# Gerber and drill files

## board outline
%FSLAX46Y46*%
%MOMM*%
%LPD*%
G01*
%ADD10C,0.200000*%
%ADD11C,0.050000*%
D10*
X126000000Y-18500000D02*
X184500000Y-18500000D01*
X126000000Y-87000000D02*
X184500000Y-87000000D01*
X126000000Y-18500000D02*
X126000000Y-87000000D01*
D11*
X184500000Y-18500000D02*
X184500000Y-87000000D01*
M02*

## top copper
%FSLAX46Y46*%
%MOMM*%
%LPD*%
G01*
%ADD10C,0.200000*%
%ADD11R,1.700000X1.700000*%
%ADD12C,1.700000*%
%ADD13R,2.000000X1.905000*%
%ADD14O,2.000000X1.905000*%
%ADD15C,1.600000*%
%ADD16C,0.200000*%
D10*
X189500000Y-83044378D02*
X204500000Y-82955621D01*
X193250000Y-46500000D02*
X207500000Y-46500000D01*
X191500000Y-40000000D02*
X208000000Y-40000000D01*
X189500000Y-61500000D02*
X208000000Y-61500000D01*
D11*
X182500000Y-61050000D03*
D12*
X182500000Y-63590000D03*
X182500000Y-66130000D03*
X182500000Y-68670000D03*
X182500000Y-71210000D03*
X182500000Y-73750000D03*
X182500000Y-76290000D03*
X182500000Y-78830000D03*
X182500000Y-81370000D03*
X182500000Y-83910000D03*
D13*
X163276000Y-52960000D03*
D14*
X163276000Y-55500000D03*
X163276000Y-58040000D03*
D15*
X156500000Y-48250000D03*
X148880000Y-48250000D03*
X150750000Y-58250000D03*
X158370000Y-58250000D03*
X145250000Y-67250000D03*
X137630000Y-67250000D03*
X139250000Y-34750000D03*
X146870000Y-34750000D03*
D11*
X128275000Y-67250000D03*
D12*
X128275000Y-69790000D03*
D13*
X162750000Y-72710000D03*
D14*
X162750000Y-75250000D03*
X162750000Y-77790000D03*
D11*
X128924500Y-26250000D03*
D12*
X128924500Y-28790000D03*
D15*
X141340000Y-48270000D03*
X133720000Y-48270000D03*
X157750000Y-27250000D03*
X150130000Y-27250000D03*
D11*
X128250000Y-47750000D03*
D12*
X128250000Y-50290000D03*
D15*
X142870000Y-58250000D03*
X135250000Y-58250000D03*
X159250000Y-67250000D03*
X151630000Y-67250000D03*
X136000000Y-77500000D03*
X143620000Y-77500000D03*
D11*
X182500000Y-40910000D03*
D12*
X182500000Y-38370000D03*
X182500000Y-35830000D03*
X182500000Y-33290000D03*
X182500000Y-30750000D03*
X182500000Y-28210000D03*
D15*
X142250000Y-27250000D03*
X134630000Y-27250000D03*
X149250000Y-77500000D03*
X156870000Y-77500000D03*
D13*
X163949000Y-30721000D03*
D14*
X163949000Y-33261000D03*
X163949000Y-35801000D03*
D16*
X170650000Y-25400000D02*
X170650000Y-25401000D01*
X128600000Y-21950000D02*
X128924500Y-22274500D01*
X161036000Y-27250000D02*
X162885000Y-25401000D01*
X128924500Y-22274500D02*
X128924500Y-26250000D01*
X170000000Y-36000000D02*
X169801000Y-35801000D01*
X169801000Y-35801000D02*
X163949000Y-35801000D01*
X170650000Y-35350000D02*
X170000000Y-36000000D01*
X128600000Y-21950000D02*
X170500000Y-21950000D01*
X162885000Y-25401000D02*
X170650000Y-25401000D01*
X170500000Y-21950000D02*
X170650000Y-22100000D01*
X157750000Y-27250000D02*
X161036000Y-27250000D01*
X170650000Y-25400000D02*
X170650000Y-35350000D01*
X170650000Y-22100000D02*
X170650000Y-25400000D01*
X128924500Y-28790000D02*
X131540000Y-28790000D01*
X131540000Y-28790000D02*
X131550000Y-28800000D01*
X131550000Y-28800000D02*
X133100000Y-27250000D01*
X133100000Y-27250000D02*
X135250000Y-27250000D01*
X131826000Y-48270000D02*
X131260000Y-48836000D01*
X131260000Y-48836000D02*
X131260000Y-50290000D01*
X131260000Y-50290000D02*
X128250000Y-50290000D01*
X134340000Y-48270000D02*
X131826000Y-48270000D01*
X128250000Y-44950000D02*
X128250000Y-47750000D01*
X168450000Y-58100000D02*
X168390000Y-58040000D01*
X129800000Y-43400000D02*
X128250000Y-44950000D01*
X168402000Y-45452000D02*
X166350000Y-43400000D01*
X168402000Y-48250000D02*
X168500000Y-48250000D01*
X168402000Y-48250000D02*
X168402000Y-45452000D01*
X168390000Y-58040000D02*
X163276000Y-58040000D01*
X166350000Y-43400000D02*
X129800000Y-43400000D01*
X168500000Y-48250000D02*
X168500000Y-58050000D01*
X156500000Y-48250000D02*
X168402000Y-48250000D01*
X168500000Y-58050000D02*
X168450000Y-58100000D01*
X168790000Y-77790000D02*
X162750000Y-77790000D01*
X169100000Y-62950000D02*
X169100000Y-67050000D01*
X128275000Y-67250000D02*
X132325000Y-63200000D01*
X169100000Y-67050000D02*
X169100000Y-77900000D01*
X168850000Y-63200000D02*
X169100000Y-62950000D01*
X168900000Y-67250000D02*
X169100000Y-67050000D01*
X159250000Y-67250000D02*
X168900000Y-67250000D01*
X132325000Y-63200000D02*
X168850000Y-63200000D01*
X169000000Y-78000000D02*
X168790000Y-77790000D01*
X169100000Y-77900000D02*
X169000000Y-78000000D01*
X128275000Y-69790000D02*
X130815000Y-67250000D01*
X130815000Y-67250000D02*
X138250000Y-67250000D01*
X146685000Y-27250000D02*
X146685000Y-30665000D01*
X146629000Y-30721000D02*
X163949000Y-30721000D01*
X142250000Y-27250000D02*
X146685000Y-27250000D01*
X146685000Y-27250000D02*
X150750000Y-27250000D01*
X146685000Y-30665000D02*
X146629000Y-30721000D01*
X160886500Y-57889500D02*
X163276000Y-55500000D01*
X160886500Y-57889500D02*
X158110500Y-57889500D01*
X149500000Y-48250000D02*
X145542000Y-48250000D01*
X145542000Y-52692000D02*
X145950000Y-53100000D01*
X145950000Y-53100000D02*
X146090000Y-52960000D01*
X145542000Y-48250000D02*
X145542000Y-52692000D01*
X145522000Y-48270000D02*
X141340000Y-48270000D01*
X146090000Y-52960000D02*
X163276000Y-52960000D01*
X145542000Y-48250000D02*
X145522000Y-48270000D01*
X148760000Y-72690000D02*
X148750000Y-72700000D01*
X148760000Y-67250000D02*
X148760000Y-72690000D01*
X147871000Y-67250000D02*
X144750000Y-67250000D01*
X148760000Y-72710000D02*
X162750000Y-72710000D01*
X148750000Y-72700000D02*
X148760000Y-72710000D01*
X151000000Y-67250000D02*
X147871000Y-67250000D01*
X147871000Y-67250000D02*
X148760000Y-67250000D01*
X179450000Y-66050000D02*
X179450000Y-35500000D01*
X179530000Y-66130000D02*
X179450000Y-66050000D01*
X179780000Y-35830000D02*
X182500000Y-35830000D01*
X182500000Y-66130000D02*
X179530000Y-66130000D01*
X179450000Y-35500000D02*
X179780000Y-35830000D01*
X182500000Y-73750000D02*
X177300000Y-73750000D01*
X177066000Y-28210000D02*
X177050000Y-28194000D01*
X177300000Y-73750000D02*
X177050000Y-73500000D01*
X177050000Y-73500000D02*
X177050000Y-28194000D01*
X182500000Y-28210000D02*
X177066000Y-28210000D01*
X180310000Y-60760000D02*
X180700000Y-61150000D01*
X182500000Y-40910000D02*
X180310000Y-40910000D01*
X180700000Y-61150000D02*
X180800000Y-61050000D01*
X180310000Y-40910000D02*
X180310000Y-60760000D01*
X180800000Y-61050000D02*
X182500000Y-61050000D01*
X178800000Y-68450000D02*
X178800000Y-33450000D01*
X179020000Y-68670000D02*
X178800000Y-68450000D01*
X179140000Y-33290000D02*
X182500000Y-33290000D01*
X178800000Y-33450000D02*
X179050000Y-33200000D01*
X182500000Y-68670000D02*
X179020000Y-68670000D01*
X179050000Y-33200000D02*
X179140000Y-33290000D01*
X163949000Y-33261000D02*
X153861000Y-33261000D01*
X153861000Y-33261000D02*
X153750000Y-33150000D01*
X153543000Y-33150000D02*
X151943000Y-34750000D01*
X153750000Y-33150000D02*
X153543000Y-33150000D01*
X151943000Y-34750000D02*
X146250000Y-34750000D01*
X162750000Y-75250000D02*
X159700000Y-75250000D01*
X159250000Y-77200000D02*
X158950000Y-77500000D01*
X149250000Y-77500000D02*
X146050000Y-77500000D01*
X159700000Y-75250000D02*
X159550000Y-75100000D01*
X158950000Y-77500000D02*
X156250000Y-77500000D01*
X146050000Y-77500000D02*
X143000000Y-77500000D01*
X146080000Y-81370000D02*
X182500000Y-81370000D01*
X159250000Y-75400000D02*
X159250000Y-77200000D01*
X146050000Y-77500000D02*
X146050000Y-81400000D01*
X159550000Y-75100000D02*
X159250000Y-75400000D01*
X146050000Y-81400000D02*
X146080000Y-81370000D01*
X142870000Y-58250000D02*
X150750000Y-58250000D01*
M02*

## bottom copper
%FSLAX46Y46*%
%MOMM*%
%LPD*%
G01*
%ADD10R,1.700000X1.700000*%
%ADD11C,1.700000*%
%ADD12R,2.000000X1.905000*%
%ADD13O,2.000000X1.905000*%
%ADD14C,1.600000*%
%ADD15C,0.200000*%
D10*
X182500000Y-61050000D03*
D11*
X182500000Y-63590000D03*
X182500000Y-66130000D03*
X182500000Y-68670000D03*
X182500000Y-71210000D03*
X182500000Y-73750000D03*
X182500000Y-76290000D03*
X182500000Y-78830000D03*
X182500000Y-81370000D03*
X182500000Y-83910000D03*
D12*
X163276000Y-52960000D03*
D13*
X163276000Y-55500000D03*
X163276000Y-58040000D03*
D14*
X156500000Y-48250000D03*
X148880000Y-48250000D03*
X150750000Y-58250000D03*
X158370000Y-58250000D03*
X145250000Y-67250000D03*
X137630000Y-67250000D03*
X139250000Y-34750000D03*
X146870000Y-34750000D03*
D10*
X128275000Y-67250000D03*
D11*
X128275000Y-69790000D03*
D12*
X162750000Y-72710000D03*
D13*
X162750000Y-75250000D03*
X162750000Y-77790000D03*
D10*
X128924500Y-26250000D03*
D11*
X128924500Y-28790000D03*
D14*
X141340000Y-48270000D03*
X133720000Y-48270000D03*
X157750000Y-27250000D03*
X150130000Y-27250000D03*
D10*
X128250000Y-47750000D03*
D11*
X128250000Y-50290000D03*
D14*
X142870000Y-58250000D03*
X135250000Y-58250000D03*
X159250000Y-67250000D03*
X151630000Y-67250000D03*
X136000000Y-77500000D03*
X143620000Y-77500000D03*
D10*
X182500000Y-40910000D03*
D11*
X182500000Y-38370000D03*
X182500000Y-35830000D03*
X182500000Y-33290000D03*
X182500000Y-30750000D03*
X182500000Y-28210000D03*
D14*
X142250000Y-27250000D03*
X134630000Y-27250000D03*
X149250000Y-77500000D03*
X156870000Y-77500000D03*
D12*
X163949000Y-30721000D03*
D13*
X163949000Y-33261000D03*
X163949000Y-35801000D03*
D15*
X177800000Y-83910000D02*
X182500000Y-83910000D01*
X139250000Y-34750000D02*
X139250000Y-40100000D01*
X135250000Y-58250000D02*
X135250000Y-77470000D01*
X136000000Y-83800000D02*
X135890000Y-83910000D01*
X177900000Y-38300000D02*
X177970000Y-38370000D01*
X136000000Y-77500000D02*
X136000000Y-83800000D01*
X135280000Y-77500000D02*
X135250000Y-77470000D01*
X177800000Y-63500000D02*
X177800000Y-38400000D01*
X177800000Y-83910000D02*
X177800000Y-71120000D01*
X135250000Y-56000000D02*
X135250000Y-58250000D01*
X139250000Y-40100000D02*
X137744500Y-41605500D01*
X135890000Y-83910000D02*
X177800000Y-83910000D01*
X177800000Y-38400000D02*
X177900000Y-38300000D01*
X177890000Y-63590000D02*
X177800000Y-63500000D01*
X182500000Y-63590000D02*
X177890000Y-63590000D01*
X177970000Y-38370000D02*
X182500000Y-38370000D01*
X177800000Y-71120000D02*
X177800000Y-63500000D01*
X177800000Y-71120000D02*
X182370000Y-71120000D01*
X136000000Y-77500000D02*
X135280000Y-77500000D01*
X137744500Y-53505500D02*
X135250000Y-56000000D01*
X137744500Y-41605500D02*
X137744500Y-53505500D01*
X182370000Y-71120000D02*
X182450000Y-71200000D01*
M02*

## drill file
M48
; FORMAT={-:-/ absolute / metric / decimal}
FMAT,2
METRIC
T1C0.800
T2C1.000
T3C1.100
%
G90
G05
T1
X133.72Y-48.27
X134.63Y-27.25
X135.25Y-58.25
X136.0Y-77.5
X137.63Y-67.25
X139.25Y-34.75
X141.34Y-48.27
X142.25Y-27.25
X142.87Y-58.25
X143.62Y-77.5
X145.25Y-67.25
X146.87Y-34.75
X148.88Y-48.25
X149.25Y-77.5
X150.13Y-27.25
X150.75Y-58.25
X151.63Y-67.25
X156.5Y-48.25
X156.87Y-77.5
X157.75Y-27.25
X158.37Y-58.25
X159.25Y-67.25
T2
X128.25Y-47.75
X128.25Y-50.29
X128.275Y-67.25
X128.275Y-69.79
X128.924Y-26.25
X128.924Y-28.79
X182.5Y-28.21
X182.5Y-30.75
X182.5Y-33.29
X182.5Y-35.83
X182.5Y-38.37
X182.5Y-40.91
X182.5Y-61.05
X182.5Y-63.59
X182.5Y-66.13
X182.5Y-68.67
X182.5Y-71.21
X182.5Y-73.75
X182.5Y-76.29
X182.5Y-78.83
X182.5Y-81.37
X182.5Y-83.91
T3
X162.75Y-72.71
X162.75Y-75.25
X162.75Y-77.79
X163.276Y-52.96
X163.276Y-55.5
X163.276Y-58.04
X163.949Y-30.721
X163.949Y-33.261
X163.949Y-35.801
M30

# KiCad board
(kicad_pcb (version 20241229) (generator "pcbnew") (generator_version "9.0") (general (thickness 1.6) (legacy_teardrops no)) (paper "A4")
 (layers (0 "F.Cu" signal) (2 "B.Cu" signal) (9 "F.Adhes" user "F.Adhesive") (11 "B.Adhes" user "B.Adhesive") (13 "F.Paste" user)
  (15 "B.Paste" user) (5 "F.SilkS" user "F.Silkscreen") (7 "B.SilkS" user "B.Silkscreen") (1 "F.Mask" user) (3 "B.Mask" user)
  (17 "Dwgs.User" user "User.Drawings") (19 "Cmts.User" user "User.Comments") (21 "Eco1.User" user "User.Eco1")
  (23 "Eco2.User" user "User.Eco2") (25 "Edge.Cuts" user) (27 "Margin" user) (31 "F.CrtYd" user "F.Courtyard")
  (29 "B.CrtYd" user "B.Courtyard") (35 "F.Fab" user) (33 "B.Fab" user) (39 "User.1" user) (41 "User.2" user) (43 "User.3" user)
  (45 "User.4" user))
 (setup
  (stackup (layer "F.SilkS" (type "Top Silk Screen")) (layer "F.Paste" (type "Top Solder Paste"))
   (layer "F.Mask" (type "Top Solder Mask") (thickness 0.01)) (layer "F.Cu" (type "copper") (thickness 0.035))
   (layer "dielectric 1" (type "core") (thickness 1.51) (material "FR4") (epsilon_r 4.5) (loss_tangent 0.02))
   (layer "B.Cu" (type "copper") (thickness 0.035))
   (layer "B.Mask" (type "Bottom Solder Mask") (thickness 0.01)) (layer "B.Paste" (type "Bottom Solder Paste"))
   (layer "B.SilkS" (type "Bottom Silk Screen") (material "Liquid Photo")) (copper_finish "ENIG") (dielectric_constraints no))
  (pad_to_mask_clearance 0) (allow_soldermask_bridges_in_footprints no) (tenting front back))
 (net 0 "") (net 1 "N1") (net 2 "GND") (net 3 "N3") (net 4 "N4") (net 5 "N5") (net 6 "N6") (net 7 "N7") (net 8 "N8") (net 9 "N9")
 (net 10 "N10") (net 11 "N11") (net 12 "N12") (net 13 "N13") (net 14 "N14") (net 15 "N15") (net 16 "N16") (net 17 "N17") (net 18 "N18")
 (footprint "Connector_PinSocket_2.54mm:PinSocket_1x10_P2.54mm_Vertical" (layer "F.Cu") (at 182.5 61.05)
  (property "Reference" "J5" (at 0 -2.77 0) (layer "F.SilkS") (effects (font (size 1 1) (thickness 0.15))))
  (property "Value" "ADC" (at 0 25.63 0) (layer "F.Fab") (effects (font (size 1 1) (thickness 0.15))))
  (pad "1" thru_hole rect (at 0 0) (size 1.7 1.7) (drill 1) (layers "*.Cu" "*.Mask") (remove_unused_layers yes) (keep_end_layers yes)
   (zone_layer_connections) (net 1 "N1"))
  (pad "2" thru_hole circle (at 0 2.54) (size 1.7 1.7) (drill 1) (layers "*.Cu" "*.Mask") (remove_unused_layers yes) (keep_end_layers yes)
   (zone_layer_connections) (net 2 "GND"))
  (pad "3" thru_hole circle (at 0 5.08) (size 1.7 1.7) (drill 1) (layers "*.Cu" "*.Mask") (remove_unused_layers yes) (keep_end_layers yes)
   (zone_layer_connections) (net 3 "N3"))
  (pad "4" thru_hole circle (at 0 7.62) (size 1.7 1.7) (drill 1) (layers "*.Cu" "*.Mask") (remove_unused_layers yes) (keep_end_layers yes)
   (zone_layer_connections) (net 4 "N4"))
  (pad "5" thru_hole circle (at 0 10.16) (size 1.7 1.7) (drill 1) (layers "*.Cu" "*.Mask") (remove_unused_layers yes) (keep_end_layers yes)
   (zone_layer_connections) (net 2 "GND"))
  (pad "6" thru_hole circle (at 0 12.7) (size 1.7 1.7) (drill 1) (layers "*.Cu" "*.Mask") (remove_unused_layers yes) (keep_end_layers yes)
   (zone_layer_connections) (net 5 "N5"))
  (pad "7" thru_hole circle (at 0 15.24) (size 1.7 1.7) (drill 1) (layers "*.Cu" "*.Mask") (remove_unused_layers yes) (keep_end_layers yes)
   (zone_layer_connections) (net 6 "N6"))
  (pad "8" thru_hole circle (at 0 17.78) (size 1.7 1.7) (drill 1) (layers "*.Cu" "*.Mask") (remove_unused_layers yes) (keep_end_layers yes)
   (zone_layer_connections) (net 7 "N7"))
  (pad "9" thru_hole circle (at 0 20.32) (size 1.7 1.7) (drill 1) (layers "*.Cu" "*.Mask") (remove_unused_layers yes) (keep_end_layers yes)
   (zone_layer_connections) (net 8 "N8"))
  (pad "10" thru_hole circle (at 0 22.86) (size 1.7 1.7) (drill 1) (layers "*.Cu" "*.Mask") (remove_unused_layers yes) (keep_end_layers yes)
   (zone_layer_connections) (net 2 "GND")))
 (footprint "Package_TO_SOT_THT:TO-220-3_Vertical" (layer "F.Cu") (at 163.276 52.96 -90)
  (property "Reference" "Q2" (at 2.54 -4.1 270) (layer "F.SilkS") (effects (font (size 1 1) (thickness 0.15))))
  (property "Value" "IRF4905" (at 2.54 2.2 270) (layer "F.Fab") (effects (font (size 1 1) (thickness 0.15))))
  (pad "1" thru_hole rect (at 0 0 270) (size 1.905 2) (drill 1.1) (layers "*.Cu" "*.Mask") (remove_unused_layers yes) (keep_end_layers yes)
   (zone_layer_connections) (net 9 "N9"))
  (pad "2" thru_hole oval (at 2.54 0 270) (size 1.905 2) (drill 1.1) (layers "*.Cu" "*.Mask") (remove_unused_layers yes)
   (keep_end_layers yes) (zone_layer_connections) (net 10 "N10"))
  (pad "3" thru_hole oval (at 5.08 0 270) (size 1.905 2) (drill 1.1) (layers "*.Cu" "*.Mask") (remove_unused_layers yes)
   (keep_end_layers yes) (zone_layer_connections) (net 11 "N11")))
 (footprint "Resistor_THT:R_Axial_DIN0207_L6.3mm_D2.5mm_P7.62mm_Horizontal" (layer "F.Cu") (at 156.5 48.25 180)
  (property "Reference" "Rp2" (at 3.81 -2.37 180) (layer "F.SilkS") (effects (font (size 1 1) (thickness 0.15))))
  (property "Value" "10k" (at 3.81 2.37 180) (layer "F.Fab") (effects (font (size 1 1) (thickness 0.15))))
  (pad "1" thru_hole circle (at 0 0 180) (size 1.6 1.6) (drill 0.8) (layers "*.Cu" "*.Mask") (remove_unused_layers no) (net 11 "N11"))
  (pad "2" thru_hole circle (at 7.62 0 180) (size 1.6 1.6) (drill 0.8) (layers "*.Cu" "*.Mask") (remove_unused_layers no) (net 9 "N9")))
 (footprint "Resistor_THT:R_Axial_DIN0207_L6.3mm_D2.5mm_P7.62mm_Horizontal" (layer "F.Cu") (at 150.75 58.25)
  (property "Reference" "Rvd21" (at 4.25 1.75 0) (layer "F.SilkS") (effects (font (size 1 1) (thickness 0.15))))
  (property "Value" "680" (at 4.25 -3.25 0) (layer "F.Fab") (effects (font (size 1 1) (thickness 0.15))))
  (pad "1" thru_hole circle (at 0 0) (size 1.6 1.6) (drill 0.8) (layers "*.Cu" "*.Mask") (remove_unused_layers no) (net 7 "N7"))
  (pad "2" thru_hole circle (at 7.62 0) (size 1.6 1.6) (drill 0.8) (layers "*.Cu" "*.Mask") (remove_unused_layers no) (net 10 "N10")))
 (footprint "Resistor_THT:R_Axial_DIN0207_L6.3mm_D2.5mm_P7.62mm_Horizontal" (layer "F.Cu") (at 145.25 67.25 180)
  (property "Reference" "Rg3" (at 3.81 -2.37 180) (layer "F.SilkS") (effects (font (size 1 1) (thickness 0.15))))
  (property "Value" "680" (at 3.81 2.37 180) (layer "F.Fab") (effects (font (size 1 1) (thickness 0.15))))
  (pad "1" thru_hole circle (at 0 0 180) (size 1.6 1.6) (drill 0.8) (layers "*.Cu" "*.Mask") (remove_unused_layers no) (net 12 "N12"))
  (pad "2" thru_hole circle (at 7.62 0 180) (size 1.6 1.6) (drill 0.8) (layers "*.Cu" "*.Mask") (remove_unused_layers no) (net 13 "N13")))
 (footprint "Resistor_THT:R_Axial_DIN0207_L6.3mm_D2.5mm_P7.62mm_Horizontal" (layer "F.Cu") (at 139.25 34.75)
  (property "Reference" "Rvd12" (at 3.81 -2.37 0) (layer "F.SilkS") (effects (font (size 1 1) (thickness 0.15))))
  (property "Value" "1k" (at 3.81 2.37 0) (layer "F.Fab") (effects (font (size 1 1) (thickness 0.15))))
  (pad "1" thru_hole circle (at 0 0) (size 1.6 1.6) (drill 0.8) (layers "*.Cu" "*.Mask") (remove_unused_layers no) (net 2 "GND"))
  (pad "2" thru_hole circle (at 7.62 0) (size 1.6 1.6) (drill 0.8) (layers "*.Cu" "*.Mask") (remove_unused_layers no) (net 6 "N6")))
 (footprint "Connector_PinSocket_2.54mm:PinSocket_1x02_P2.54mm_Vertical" (layer "F.Cu") (at 128.275 67.25)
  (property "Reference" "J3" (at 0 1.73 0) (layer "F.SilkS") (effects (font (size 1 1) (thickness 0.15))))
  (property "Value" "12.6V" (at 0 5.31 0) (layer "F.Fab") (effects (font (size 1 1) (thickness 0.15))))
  (pad "1" thru_hole rect (at 0 0) (size 1.7 1.7) (drill 1) (layers "*.Cu" "*.Mask") (remove_unused_layers yes) (keep_end_layers yes)
   (zone_layer_connections) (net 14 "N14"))
  (pad "2" thru_hole circle (at 0 2.54) (size 1.7 1.7) (drill 1) (layers "*.Cu" "*.Mask") (remove_unused_layers yes) (keep_end_layers yes)
   (zone_layer_connections) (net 13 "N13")))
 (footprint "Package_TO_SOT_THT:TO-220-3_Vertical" (layer "F.Cu") (at 162.75 72.71 -90)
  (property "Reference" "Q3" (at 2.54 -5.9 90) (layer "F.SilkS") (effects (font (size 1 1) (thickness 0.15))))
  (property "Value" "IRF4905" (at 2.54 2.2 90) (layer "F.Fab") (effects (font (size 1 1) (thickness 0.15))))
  (pad "1" thru_hole rect (at 0 0 270) (size 1.905 2) (drill 1.1) (layers "*.Cu" "*.Mask") (remove_unused_layers yes) (keep_end_layers yes)
   (zone_layer_connections) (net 12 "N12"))
  (pad "2" thru_hole oval (at 2.54 0 270) (size 1.905 2) (drill 1.1) (layers "*.Cu" "*.Mask") (remove_unused_layers yes)
   (keep_end_layers yes) (zone_layer_connections) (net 8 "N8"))
  (pad "3" thru_hole oval (at 5.08 0 270) (size 1.905 2) (drill 1.1) (layers "*.Cu" "*.Mask") (remove_unused_layers yes)
   (keep_end_layers yes) (zone_layer_connections) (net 14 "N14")))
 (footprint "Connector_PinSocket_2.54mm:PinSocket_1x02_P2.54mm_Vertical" (layer "F.Cu") (at 128.9245 26.25)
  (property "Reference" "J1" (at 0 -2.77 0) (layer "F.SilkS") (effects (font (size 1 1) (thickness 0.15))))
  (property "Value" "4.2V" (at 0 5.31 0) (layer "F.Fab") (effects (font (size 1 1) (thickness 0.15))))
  (pad "1" thru_hole rect (at 0 0) (size 1.7 1.7) (drill 1) (layers "*.Cu" "*.Mask") (remove_unused_layers yes) (keep_end_layers yes)
   (zone_layer_connections) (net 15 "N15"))
  (pad "2" thru_hole circle (at 0 2.54) (size 1.7 1.7) (drill 1) (layers "*.Cu" "*.Mask") (remove_unused_layers yes) (keep_end_layers yes)
   (zone_layer_connections) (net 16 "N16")))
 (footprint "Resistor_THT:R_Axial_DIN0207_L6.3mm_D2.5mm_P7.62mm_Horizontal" (layer "F.Cu") (at 141.34 48.27 180)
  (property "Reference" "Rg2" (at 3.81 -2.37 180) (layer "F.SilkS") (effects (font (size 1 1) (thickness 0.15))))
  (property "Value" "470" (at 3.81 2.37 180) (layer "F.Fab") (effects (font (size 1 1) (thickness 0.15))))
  (pad "1" thru_hole circle (at 0 0 180) (size 1.6 1.6) (drill 0.8) (layers "*.Cu" "*.Mask") (remove_unused_layers no) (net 9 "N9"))
  (pad "2" thru_hole circle (at 7.62 0 180) (size 1.6 1.6) (drill 0.8) (layers "*.Cu" "*.Mask") (remove_unused_layers no) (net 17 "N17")))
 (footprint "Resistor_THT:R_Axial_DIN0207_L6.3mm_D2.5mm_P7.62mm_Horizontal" (layer "F.Cu") (at 157.75 27.25 180)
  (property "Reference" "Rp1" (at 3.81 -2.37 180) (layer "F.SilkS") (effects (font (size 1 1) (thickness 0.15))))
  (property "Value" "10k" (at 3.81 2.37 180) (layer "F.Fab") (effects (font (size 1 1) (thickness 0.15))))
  (pad "1" thru_hole circle (at 0 0 180) (size 1.6 1.6) (drill 0.8) (layers "*.Cu" "*.Mask") (remove_unused_layers no) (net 15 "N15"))
  (pad "2" thru_hole circle (at 7.62 0 180) (size 1.6 1.6) (drill 0.8) (layers "*.Cu" "*.Mask") (remove_unused_layers no) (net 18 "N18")))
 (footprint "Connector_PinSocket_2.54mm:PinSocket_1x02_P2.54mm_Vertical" (layer "F.Cu") (at 128.25 47.75)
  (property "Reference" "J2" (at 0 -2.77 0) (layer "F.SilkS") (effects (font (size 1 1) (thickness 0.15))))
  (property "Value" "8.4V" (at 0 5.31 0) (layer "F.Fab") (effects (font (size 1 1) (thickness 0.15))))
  (pad "1" thru_hole rect (at 0 0) (size 1.7 1.7) (drill 1) (layers "*.Cu" "*.Mask") (remove_unused_layers yes) (keep_end_layers yes)
   (zone_layer_connections) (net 11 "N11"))
  (pad "2" thru_hole circle (at 0 2.54) (size 1.7 1.7) (drill 1) (layers "*.Cu" "*.Mask") (remove_unused_layers yes) (keep_end_layers yes)
   (zone_layer_connections) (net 17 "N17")))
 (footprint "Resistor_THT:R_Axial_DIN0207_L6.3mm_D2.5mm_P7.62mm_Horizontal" (layer "F.Cu") (at 142.87 58.25 180)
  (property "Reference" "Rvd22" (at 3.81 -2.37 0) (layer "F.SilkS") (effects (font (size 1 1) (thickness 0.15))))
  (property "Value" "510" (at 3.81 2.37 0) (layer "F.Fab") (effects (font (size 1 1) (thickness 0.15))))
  (pad "1" thru_hole circle (at 0 0 180) (size 1.6 1.6) (drill 0.8) (layers "*.Cu" "*.Mask") (remove_unused_layers no) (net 7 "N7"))
  (pad "2" thru_hole circle (at 7.62 0 180) (size 1.6 1.6) (drill 0.8) (layers "*.Cu" "*.Mask") (remove_unused_layers no) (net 2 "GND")))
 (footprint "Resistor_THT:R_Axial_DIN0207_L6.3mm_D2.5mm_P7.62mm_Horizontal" (layer "F.Cu") (at 159.25 67.25 180)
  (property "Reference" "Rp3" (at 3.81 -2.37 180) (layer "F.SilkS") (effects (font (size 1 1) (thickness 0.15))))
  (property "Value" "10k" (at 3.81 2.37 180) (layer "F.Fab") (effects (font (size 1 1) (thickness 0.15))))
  (pad "1" thru_hole circle (at 0 0 180) (size 1.6 1.6) (drill 0.8) (layers "*.Cu" "*.Mask") (remove_unused_layers no) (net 14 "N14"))
  (pad "2" thru_hole circle (at 7.62 0 180) (size 1.6 1.6) (drill 0.8) (layers "*.Cu" "*.Mask") (remove_unused_layers no) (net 12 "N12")))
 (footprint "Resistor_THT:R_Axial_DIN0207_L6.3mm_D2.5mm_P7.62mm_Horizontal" (layer "F.Cu") (at 136 77.5)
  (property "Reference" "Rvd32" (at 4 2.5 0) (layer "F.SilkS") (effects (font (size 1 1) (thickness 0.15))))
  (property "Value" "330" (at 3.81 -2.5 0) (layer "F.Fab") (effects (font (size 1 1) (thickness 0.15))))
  (pad "1" thru_hole circle (at 0 0) (size 1.6 1.6) (drill 0.8) (layers "*.Cu" "*.Mask") (remove_unused_layers no) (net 2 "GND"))
  (pad "2" thru_hole circle (at 7.62 0) (size 1.6 1.6) (drill 0.8) (layers "*.Cu" "*.Mask") (remove_unused_layers no) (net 8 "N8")))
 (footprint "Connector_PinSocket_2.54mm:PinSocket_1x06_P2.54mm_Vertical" (layer "F.Cu") (at 182.5 40.91 180)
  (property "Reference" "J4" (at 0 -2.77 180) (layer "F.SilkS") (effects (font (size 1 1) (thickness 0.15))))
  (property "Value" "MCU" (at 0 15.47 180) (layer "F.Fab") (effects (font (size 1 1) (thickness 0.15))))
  (pad "1" thru_hole rect (at 0 0 180) (size 1.7 1.7) (drill 1) (layers "*.Cu" "*.Mask") (remove_unused_layers yes) (keep_end_layers yes)
   (zone_layer_connections) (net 1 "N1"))
  (pad "2" thru_hole circle (at 0 2.54 180) (size 1.7 1.7) (drill 1) (layers "*.Cu" "*.Mask") (remove_unused_layers yes)
   (keep_end_layers yes) (zone_layer_connections) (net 2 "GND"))
  (pad "3" thru_hole circle (at 0 5.08 180) (size 1.7 1.7) (drill 1) (layers "*.Cu" "*.Mask") (remove_unused_layers yes)
   (keep_end_layers yes) (zone_layer_connections) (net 3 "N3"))
  (pad "4" thru_hole circle (at 0 7.62 180) (size 1.7 1.7) (drill 1) (layers "*.Cu" "*.Mask") (remove_unused_layers yes)
   (keep_end_layers yes) (zone_layer_connections) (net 4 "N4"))
  (pad "5" thru_hole circle (at 0 10.16 180) (size 1.7 1.7) (drill 1) (layers "*.Cu" "*.Mask") (remove_unused_layers yes)
   (keep_end_layers yes) (zone_layer_connections) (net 2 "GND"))
  (pad "6" thru_hole circle (at 0 12.7 180) (size 1.7 1.7) (drill 1) (layers "*.Cu" "*.Mask") (remove_unused_layers yes)
   (keep_end_layers yes) (zone_layer_connections) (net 5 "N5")))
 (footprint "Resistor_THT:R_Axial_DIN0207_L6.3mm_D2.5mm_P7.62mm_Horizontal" (layer "F.Cu") (at 142.25 27.25 180)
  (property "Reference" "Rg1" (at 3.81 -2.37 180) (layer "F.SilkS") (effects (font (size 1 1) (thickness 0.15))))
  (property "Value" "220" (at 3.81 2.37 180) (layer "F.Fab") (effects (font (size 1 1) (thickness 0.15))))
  (pad "1" thru_hole circle (at 0 0 180) (size 1.6 1.6) (drill 0.8) (layers "*.Cu" "*.Mask") (remove_unused_layers no) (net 18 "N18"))
  (pad "2" thru_hole circle (at 7.62 0 180) (size 1.6 1.6) (drill 0.8) (layers "*.Cu" "*.Mask") (remove_unused_layers no) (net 16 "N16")))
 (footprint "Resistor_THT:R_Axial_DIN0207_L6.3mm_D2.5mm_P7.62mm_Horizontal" (layer "F.Cu") (at 149.25 77.5)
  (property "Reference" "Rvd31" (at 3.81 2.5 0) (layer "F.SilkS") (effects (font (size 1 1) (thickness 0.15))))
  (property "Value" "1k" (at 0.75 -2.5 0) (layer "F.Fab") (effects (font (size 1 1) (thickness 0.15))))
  (pad "1" thru_hole circle (at 0 0) (size 1.6 1.6) (drill 0.8) (layers "*.Cu" "*.Mask") (remove_unused_layers no) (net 8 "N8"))
  (pad "2" thru_hole circle (at 7.62 0) (size 1.6 1.6) (drill 0.8) (layers "*.Cu" "*.Mask") (remove_unused_layers no) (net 8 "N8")))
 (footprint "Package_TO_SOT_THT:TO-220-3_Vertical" (layer "F.Cu") (at 163.949 30.721 -90)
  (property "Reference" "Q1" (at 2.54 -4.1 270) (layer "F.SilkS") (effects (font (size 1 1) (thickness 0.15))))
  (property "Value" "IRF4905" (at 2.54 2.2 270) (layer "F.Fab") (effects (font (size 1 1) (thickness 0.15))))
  (pad "1" thru_hole rect (at 0 0 270) (size 1.905 2) (drill 1.1) (layers "*.Cu" "*.Mask") (remove_unused_layers yes) (keep_end_layers yes)
   (zone_layer_connections) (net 18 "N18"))
  (pad "2" thru_hole oval (at 2.54 0 270) (size 1.905 2) (drill 1.1) (layers "*.Cu" "*.Mask") (remove_unused_layers yes)
   (keep_end_layers yes) (zone_layer_connections) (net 6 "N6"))
  (pad "3" thru_hole oval (at 5.08 0 270) (size 1.905 2) (drill 1.1) (layers "*.Cu" "*.Mask") (remove_unused_layers yes)
   (keep_end_layers yes) (zone_layer_connections) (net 15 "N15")))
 (gr_line (start 189.5 83.044378) (end 204.5 82.955621) (stroke (width 0.2) (type default)) (layer "F.Cu"))
 (gr_line (start 193.25 46.5) (end 207.5 46.5) (stroke (width 0.2) (type default)) (layer "F.Cu"))
 (gr_line (start 191.5 40) (end 208 40) (stroke (width 0.2) (type default)) (layer "F.Cu"))
 (gr_line (start 189.5 61.5) (end 208 61.5) (stroke (width 0.2) (type default)) (layer "F.Cu"))
 (gr_line (start 126 18.5) (end 184.5 18.5) (stroke (width 0.2) (type solid)) (layer "Edge.Cuts"))
 (gr_line (start 126 87) (end 184.5 87) (stroke (width 0.2) (type solid)) (layer "Edge.Cuts"))
 (gr_line (start 126 18.5) (end 126 87) (stroke (width 0.2) (type solid)) (layer "Edge.Cuts"))
 (gr_line (start 184.5 18.5) (end 184.5 87) (stroke (width 0.05) (type solid)) (layer "Edge.Cuts"))
 (segment (start 170.65 25.4) (end 170.65 25.401) (width 0.2) (layer "F.Cu") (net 15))
 (segment (start 128.6 21.95) (end 128.9245 22.2745) (width 0.2) (layer "F.Cu") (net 15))
 (segment (start 161.036 27.25) (end 162.885 25.401) (width 0.2) (layer "F.Cu") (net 15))
 (segment (start 128.9245 22.2745) (end 128.9245 26.25) (width 0.2) (layer "F.Cu") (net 15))
 (segment (start 170 36) (end 169.801 35.801) (width 0.2) (layer "F.Cu") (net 15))
 (segment (start 169.801 35.801) (end 163.949 35.801) (width 0.2) (layer "F.Cu") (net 15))
 (segment (start 170.65 35.35) (end 170 36) (width 0.2) (layer "F.Cu") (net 15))
 (segment (start 128.6 21.95) (end 170.5 21.95) (width 0.2) (layer "F.Cu") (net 15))
 (segment (start 162.885 25.401) (end 170.65 25.401) (width 0.2) (layer "F.Cu") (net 15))
 (segment (start 170.5 21.95) (end 170.65 22.1) (width 0.2) (layer "F.Cu") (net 15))
 (segment (start 157.75 27.25) (end 161.036 27.25) (width 0.2) (layer "F.Cu") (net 15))
 (segment (start 170.65 25.4) (end 170.65 35.35) (width 0.2) (layer "F.Cu") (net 15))
 (segment (start 170.65 22.1) (end 170.65 25.4) (width 0.2) (layer "F.Cu") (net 15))
 (segment (start 128.9245 28.79) (end 131.54 28.79) (width 0.2) (layer "F.Cu") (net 16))
 (segment (start 131.54 28.79) (end 131.55 28.8) (width 0.2) (layer "F.Cu") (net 16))
 (segment (start 131.55 28.8) (end 133.1 27.25) (width 0.2) (layer "F.Cu") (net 16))
 (segment (start 133.1 27.25) (end 135.25 27.25) (width 0.2) (layer "F.Cu") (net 16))
 (segment (start 131.826 48.27) (end 131.26 48.836) (width 0.2) (layer "F.Cu") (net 17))
 (segment (start 131.26 48.836) (end 131.26 50.29) (width 0.2) (layer "F.Cu") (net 17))
 (segment (start 131.26 50.29) (end 128.25 50.29) (width 0.2) (layer "F.Cu") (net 17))
 (segment (start 134.34 48.27) (end 131.826 48.27) (width 0.2) (layer "F.Cu") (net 17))
 (segment (start 128.25 44.95) (end 128.25 47.75) (width 0.2) (layer "F.Cu") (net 11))
 (segment (start 168.45 58.1) (end 168.39 58.04) (width 0.2) (layer "F.Cu") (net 11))
 (segment (start 129.8 43.4) (end 128.25 44.95) (width 0.2) (layer "F.Cu") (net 11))
 (segment (start 168.402 45.452) (end 166.35 43.4) (width 0.2) (layer "F.Cu") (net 11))
 (segment (start 168.402 48.25) (end 168.5 48.25) (width 0.2) (layer "F.Cu") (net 11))
 (segment (start 168.402 48.25) (end 168.402 45.452) (width 0.2) (layer "F.Cu") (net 11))
 (segment (start 168.39 58.04) (end 163.276 58.04) (width 0.2) (layer "F.Cu") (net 11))
 (segment (start 166.35 43.4) (end 129.8 43.4) (width 0.2) (layer "F.Cu") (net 11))
 (segment (start 168.5 48.25) (end 168.5 58.05) (width 0.2) (layer "F.Cu") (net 11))
 (segment (start 156.5 48.25) (end 168.402 48.25) (width 0.2) (layer "F.Cu") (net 11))
 (segment (start 168.5 58.05) (end 168.45 58.1) (width 0.2) (layer "F.Cu") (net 11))
 (segment (start 168.79 77.79) (end 162.75 77.79) (width 0.2) (layer "F.Cu") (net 14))
 (segment (start 169.1 62.95) (end 169.1 67.05) (width 0.2) (layer "F.Cu") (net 14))
 (segment (start 128.275 67.25) (end 132.325 63.2) (width 0.2) (layer "F.Cu") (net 14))
 (segment (start 169.1 67.05) (end 169.1 77.9) (width 0.2) (layer "F.Cu") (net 14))
 (segment (start 168.85 63.2) (end 169.1 62.95) (width 0.2) (layer "F.Cu") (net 14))
 (segment (start 168.9 67.25) (end 169.1 67.05) (width 0.2) (layer "F.Cu") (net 14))
 (segment (start 159.25 67.25) (end 168.9 67.25) (width 0.2) (layer "F.Cu") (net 14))
 (segment (start 132.325 63.2) (end 168.85 63.2) (width 0.2) (layer "F.Cu") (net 14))
 (segment (start 169 78) (end 168.79 77.79) (width 0.2) (layer "F.Cu") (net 14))
 (segment (start 169.1 77.9) (end 169 78) (width 0.2) (layer "F.Cu") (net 14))
 (segment (start 128.275 69.79) (end 130.815 67.25) (width 0.2) (layer "F.Cu") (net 13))
 (segment (start 130.815 67.25) (end 138.25 67.25) (width 0.2) (layer "F.Cu") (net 13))
 (segment (start 146.685 27.25) (end 146.685 30.665) (width 0.2) (layer "F.Cu") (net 18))
 (segment (start 146.629 30.721) (end 163.949 30.721) (width 0.2) (layer "F.Cu") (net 18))
 (segment (start 142.25 27.25) (end 146.685 27.25) (width 0.2) (layer "F.Cu") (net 18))
 (segment (start 146.685 27.25) (end 150.75 27.25) (width 0.2) (layer "F.Cu") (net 18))
 (segment (start 146.685 30.665) (end 146.629 30.721) (width 0.2) (layer "F.Cu") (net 18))
 (segment (start 160.8865 57.8895) (end 163.276 55.5) (width 0.2) (layer "F.Cu") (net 10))
 (segment (start 160.8865 57.8895) (end 158.1105 57.8895) (width 0.2) (layer "F.Cu") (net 10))
 (segment (start 149.5 48.25) (end 145.542 48.25) (width 0.2) (layer "F.Cu") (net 9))
 (segment (start 145.542 52.692) (end 145.95 53.1) (width 0.2) (layer "F.Cu") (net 9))
 (segment (start 145.95 53.1) (end 146.09 52.96) (width 0.2) (layer "F.Cu") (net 9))
 (segment (start 145.542 48.25) (end 145.542 52.692) (width 0.2) (layer "F.Cu") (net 9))
 (segment (start 145.522 48.27) (end 141.34 48.27) (width 0.2) (layer "F.Cu") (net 9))
 (segment (start 146.09 52.96) (end 163.276 52.96) (width 0.2) (layer "F.Cu") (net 9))
 (segment (start 145.542 48.25) (end 145.522 48.27) (width 0.2) (layer "F.Cu") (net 9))
 (segment (start 148.76 72.69) (end 148.75 72.7) (width 0.2) (layer "F.Cu") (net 12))
 (segment (start 148.76 67.25) (end 148.76 72.69) (width 0.2) (layer "F.Cu") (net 12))
 (segment (start 147.871 67.25) (end 144.75 67.25) (width 0.2) (layer "F.Cu") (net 12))
 (segment (start 148.76 72.71) (end 162.75 72.71) (width 0.2) (layer "F.Cu") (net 12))
 (segment (start 148.75 72.7) (end 148.76 72.71) (width 0.2) (layer "F.Cu") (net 12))
 (segment (start 151 67.25) (end 147.871 67.25) (width 0.2) (layer "F.Cu") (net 12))
 (segment (start 147.871 67.25) (end 148.76 67.25) (width 0.2) (layer "F.Cu") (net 12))
 (segment (start 179.45 66.05) (end 179.45 35.5) (width 0.2) (layer "F.Cu") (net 3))
 (segment (start 179.53 66.13) (end 179.45 66.05) (width 0.2) (layer "F.Cu") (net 3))
 (segment (start 179.78 35.83) (end 182.5 35.83) (width 0.2) (layer "F.Cu") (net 3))
 (segment (start 182.5 66.13) (end 179.53 66.13) (width 0.2) (layer "F.Cu") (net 3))
 (segment (start 179.45 35.5) (end 179.78 35.83) (width 0.2) (layer "F.Cu") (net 3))
 (segment (start 182.5 73.75) (end 177.3 73.75) (width 0.2) (layer "F.Cu") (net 5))
 (segment (start 177.066 28.21) (end 177.05 28.194) (width 0.2) (layer "F.Cu") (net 5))
 (segment (start 177.3 73.75) (end 177.05 73.5) (width 0.2) (layer "F.Cu") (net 5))
 (segment (start 177.05 73.5) (end 177.05 28.194) (width 0.2) (layer "F.Cu") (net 5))
 (segment (start 182.5 28.21) (end 177.066 28.21) (width 0.2) (layer "F.Cu") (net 5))
 (segment (start 180.31 60.76) (end 180.7 61.15) (width 0.2) (layer "F.Cu") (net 1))
 (segment (start 182.5 40.91) (end 180.31 40.91) (width 0.2) (layer "F.Cu") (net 1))
 (segment (start 180.7 61.15) (end 180.8 61.05) (width 0.2) (layer "F.Cu") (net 1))
 (segment (start 180.31 40.91) (end 180.31 60.76) (width 0.2) (layer "F.Cu") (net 1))
 (segment (start 180.8 61.05) (end 182.5 61.05) (width 0.2) (layer "F.Cu") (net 1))
 (segment (start 178.8 68.45) (end 178.8 33.45) (width 0.2) (layer "F.Cu") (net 4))
 (segment (start 179.02 68.67) (end 178.8 68.45) (width 0.2) (layer "F.Cu") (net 4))
 (segment (start 179.14 33.29) (end 182.5 33.29) (width 0.2) (layer "F.Cu") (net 4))
 (segment (start 178.8 33.45) (end 179.05 33.2) (width 0.2) (layer "F.Cu") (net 4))
 (segment (start 182.5 68.67) (end 179.02 68.67) (width 0.2) (layer "F.Cu") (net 4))
 (segment (start 179.05 33.2) (end 179.14 33.29) (width 0.2) (layer "F.Cu") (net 4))
 (segment (start 177.8 83.91) (end 182.5 83.91) (width 0.2) (layer "B.Cu") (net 2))
 (segment (start 139.25 34.75) (end 139.25 40.1) (width 0.2) (layer "B.Cu") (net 2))
 (segment (start 135.25 58.25) (end 135.25 77.47) (width 0.2) (layer "B.Cu") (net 2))
 (segment (start 136 83.8) (end 135.89 83.91) (width 0.2) (layer "B.Cu") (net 2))
 (segment (start 177.9 38.3) (end 177.97 38.37) (width 0.2) (layer "B.Cu") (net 2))
 (segment (start 136 77.5) (end 136 83.8) (width 0.2) (layer "B.Cu") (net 2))
 (segment (start 135.28 77.5) (end 135.25 77.47) (width 0.2) (layer "B.Cu") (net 2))
 (segment (start 177.8 63.5) (end 177.8 38.4) (width 0.2) (layer "B.Cu") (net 2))
 (segment (start 177.8 83.91) (end 177.8 71.12) (width 0.2) (layer "B.Cu") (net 2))
 (segment (start 135.25 56) (end 135.25 58.25) (width 0.2) (layer "B.Cu") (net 2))
 (segment (start 139.25 40.1) (end 137.7445 41.6055) (width 0.2) (layer "B.Cu") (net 2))
 (segment (start 135.89 83.91) (end 177.8 83.91) (width 0.2) (layer "B.Cu") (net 2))
 (segment (start 177.8 38.4) (end 177.9 38.3) (width 0.2) (layer "B.Cu") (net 2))
 (segment (start 177.89 63.59) (end 177.8 63.5) (width 0.2) (layer "B.Cu") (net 2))
 (segment (start 182.5 63.59) (end 177.89 63.59) (width 0.2) (layer "B.Cu") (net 2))
 (segment (start 177.97 38.37) (end 182.5 38.37) (width 0.2) (layer "B.Cu") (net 2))
 (segment (start 177.8 71.12) (end 177.8 63.5) (width 0.2) (layer "B.Cu") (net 2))
 (segment (start 177.8 71.12) (end 182.37 71.12) (width 0.2) (layer "B.Cu") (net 2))
 (segment (start 136 77.5) (end 135.28 77.5) (width 0.2) (layer "B.Cu") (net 2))
 (segment (start 137.7445 53.5055) (end 135.25 56) (width 0.2) (layer "B.Cu") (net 2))
 (segment (start 137.7445 41.6055) (end 137.7445 53.5055) (width 0.2) (layer "B.Cu") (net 2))
 (segment (start 182.37 71.12) (end 182.45 71.2) (width 0.2) (layer "B.Cu") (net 2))
 (segment (start 163.949 33.261) (end 153.861 33.261) (width 0.2) (layer "F.Cu") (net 6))
 (segment (start 153.861 33.261) (end 153.75 33.15) (width 0.2) (layer "F.Cu") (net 6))
 (segment (start 153.543 33.15) (end 151.943 34.75) (width 0.2) (layer "F.Cu") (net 6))
 (segment (start 153.75 33.15) (end 153.543 33.15) (width 0.2) (layer "F.Cu") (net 6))
 (segment (start 151.943 34.75) (end 146.25 34.75) (width 0.2) (layer "F.Cu") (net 6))
 (segment (start 162.75 75.25) (end 159.7 75.25) (width 0.2) (layer "F.Cu") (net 8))
 (segment (start 159.25 77.2) (end 158.95 77.5) (width 0.2) (layer "F.Cu") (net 8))
 (segment (start 149.25 77.5) (end 146.05 77.5) (width 0.2) (layer "F.Cu") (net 8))
 (segment (start 159.7 75.25) (end 159.55 75.1) (width 0.2) (layer "F.Cu") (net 8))
 (segment (start 158.95 77.5) (end 156.25 77.5) (width 0.2) (layer "F.Cu") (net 8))
 (segment (start 146.05 77.5) (end 143 77.5) (width 0.2) (layer "F.Cu") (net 8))
 (segment (start 146.08 81.37) (end 182.5 81.37) (width 0.2) (layer "F.Cu") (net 8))
 (segment (start 159.25 75.4) (end 159.25 77.2) (width 0.2) (layer "F.Cu") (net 8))
 (segment (start 146.05 77.5) (end 146.05 81.4) (width 0.2) (layer "F.Cu") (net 8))
 (segment (start 159.55 75.1) (end 159.25 75.4) (width 0.2) (layer "F.Cu") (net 8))
 (segment (start 146.05 81.4) (end 146.08 81.37) (width 0.2) (layer "F.Cu") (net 8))
 (segment (start 142.87 58.25) (end 150.75 58.25) (width 0.2) (layer "F.Cu") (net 7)))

